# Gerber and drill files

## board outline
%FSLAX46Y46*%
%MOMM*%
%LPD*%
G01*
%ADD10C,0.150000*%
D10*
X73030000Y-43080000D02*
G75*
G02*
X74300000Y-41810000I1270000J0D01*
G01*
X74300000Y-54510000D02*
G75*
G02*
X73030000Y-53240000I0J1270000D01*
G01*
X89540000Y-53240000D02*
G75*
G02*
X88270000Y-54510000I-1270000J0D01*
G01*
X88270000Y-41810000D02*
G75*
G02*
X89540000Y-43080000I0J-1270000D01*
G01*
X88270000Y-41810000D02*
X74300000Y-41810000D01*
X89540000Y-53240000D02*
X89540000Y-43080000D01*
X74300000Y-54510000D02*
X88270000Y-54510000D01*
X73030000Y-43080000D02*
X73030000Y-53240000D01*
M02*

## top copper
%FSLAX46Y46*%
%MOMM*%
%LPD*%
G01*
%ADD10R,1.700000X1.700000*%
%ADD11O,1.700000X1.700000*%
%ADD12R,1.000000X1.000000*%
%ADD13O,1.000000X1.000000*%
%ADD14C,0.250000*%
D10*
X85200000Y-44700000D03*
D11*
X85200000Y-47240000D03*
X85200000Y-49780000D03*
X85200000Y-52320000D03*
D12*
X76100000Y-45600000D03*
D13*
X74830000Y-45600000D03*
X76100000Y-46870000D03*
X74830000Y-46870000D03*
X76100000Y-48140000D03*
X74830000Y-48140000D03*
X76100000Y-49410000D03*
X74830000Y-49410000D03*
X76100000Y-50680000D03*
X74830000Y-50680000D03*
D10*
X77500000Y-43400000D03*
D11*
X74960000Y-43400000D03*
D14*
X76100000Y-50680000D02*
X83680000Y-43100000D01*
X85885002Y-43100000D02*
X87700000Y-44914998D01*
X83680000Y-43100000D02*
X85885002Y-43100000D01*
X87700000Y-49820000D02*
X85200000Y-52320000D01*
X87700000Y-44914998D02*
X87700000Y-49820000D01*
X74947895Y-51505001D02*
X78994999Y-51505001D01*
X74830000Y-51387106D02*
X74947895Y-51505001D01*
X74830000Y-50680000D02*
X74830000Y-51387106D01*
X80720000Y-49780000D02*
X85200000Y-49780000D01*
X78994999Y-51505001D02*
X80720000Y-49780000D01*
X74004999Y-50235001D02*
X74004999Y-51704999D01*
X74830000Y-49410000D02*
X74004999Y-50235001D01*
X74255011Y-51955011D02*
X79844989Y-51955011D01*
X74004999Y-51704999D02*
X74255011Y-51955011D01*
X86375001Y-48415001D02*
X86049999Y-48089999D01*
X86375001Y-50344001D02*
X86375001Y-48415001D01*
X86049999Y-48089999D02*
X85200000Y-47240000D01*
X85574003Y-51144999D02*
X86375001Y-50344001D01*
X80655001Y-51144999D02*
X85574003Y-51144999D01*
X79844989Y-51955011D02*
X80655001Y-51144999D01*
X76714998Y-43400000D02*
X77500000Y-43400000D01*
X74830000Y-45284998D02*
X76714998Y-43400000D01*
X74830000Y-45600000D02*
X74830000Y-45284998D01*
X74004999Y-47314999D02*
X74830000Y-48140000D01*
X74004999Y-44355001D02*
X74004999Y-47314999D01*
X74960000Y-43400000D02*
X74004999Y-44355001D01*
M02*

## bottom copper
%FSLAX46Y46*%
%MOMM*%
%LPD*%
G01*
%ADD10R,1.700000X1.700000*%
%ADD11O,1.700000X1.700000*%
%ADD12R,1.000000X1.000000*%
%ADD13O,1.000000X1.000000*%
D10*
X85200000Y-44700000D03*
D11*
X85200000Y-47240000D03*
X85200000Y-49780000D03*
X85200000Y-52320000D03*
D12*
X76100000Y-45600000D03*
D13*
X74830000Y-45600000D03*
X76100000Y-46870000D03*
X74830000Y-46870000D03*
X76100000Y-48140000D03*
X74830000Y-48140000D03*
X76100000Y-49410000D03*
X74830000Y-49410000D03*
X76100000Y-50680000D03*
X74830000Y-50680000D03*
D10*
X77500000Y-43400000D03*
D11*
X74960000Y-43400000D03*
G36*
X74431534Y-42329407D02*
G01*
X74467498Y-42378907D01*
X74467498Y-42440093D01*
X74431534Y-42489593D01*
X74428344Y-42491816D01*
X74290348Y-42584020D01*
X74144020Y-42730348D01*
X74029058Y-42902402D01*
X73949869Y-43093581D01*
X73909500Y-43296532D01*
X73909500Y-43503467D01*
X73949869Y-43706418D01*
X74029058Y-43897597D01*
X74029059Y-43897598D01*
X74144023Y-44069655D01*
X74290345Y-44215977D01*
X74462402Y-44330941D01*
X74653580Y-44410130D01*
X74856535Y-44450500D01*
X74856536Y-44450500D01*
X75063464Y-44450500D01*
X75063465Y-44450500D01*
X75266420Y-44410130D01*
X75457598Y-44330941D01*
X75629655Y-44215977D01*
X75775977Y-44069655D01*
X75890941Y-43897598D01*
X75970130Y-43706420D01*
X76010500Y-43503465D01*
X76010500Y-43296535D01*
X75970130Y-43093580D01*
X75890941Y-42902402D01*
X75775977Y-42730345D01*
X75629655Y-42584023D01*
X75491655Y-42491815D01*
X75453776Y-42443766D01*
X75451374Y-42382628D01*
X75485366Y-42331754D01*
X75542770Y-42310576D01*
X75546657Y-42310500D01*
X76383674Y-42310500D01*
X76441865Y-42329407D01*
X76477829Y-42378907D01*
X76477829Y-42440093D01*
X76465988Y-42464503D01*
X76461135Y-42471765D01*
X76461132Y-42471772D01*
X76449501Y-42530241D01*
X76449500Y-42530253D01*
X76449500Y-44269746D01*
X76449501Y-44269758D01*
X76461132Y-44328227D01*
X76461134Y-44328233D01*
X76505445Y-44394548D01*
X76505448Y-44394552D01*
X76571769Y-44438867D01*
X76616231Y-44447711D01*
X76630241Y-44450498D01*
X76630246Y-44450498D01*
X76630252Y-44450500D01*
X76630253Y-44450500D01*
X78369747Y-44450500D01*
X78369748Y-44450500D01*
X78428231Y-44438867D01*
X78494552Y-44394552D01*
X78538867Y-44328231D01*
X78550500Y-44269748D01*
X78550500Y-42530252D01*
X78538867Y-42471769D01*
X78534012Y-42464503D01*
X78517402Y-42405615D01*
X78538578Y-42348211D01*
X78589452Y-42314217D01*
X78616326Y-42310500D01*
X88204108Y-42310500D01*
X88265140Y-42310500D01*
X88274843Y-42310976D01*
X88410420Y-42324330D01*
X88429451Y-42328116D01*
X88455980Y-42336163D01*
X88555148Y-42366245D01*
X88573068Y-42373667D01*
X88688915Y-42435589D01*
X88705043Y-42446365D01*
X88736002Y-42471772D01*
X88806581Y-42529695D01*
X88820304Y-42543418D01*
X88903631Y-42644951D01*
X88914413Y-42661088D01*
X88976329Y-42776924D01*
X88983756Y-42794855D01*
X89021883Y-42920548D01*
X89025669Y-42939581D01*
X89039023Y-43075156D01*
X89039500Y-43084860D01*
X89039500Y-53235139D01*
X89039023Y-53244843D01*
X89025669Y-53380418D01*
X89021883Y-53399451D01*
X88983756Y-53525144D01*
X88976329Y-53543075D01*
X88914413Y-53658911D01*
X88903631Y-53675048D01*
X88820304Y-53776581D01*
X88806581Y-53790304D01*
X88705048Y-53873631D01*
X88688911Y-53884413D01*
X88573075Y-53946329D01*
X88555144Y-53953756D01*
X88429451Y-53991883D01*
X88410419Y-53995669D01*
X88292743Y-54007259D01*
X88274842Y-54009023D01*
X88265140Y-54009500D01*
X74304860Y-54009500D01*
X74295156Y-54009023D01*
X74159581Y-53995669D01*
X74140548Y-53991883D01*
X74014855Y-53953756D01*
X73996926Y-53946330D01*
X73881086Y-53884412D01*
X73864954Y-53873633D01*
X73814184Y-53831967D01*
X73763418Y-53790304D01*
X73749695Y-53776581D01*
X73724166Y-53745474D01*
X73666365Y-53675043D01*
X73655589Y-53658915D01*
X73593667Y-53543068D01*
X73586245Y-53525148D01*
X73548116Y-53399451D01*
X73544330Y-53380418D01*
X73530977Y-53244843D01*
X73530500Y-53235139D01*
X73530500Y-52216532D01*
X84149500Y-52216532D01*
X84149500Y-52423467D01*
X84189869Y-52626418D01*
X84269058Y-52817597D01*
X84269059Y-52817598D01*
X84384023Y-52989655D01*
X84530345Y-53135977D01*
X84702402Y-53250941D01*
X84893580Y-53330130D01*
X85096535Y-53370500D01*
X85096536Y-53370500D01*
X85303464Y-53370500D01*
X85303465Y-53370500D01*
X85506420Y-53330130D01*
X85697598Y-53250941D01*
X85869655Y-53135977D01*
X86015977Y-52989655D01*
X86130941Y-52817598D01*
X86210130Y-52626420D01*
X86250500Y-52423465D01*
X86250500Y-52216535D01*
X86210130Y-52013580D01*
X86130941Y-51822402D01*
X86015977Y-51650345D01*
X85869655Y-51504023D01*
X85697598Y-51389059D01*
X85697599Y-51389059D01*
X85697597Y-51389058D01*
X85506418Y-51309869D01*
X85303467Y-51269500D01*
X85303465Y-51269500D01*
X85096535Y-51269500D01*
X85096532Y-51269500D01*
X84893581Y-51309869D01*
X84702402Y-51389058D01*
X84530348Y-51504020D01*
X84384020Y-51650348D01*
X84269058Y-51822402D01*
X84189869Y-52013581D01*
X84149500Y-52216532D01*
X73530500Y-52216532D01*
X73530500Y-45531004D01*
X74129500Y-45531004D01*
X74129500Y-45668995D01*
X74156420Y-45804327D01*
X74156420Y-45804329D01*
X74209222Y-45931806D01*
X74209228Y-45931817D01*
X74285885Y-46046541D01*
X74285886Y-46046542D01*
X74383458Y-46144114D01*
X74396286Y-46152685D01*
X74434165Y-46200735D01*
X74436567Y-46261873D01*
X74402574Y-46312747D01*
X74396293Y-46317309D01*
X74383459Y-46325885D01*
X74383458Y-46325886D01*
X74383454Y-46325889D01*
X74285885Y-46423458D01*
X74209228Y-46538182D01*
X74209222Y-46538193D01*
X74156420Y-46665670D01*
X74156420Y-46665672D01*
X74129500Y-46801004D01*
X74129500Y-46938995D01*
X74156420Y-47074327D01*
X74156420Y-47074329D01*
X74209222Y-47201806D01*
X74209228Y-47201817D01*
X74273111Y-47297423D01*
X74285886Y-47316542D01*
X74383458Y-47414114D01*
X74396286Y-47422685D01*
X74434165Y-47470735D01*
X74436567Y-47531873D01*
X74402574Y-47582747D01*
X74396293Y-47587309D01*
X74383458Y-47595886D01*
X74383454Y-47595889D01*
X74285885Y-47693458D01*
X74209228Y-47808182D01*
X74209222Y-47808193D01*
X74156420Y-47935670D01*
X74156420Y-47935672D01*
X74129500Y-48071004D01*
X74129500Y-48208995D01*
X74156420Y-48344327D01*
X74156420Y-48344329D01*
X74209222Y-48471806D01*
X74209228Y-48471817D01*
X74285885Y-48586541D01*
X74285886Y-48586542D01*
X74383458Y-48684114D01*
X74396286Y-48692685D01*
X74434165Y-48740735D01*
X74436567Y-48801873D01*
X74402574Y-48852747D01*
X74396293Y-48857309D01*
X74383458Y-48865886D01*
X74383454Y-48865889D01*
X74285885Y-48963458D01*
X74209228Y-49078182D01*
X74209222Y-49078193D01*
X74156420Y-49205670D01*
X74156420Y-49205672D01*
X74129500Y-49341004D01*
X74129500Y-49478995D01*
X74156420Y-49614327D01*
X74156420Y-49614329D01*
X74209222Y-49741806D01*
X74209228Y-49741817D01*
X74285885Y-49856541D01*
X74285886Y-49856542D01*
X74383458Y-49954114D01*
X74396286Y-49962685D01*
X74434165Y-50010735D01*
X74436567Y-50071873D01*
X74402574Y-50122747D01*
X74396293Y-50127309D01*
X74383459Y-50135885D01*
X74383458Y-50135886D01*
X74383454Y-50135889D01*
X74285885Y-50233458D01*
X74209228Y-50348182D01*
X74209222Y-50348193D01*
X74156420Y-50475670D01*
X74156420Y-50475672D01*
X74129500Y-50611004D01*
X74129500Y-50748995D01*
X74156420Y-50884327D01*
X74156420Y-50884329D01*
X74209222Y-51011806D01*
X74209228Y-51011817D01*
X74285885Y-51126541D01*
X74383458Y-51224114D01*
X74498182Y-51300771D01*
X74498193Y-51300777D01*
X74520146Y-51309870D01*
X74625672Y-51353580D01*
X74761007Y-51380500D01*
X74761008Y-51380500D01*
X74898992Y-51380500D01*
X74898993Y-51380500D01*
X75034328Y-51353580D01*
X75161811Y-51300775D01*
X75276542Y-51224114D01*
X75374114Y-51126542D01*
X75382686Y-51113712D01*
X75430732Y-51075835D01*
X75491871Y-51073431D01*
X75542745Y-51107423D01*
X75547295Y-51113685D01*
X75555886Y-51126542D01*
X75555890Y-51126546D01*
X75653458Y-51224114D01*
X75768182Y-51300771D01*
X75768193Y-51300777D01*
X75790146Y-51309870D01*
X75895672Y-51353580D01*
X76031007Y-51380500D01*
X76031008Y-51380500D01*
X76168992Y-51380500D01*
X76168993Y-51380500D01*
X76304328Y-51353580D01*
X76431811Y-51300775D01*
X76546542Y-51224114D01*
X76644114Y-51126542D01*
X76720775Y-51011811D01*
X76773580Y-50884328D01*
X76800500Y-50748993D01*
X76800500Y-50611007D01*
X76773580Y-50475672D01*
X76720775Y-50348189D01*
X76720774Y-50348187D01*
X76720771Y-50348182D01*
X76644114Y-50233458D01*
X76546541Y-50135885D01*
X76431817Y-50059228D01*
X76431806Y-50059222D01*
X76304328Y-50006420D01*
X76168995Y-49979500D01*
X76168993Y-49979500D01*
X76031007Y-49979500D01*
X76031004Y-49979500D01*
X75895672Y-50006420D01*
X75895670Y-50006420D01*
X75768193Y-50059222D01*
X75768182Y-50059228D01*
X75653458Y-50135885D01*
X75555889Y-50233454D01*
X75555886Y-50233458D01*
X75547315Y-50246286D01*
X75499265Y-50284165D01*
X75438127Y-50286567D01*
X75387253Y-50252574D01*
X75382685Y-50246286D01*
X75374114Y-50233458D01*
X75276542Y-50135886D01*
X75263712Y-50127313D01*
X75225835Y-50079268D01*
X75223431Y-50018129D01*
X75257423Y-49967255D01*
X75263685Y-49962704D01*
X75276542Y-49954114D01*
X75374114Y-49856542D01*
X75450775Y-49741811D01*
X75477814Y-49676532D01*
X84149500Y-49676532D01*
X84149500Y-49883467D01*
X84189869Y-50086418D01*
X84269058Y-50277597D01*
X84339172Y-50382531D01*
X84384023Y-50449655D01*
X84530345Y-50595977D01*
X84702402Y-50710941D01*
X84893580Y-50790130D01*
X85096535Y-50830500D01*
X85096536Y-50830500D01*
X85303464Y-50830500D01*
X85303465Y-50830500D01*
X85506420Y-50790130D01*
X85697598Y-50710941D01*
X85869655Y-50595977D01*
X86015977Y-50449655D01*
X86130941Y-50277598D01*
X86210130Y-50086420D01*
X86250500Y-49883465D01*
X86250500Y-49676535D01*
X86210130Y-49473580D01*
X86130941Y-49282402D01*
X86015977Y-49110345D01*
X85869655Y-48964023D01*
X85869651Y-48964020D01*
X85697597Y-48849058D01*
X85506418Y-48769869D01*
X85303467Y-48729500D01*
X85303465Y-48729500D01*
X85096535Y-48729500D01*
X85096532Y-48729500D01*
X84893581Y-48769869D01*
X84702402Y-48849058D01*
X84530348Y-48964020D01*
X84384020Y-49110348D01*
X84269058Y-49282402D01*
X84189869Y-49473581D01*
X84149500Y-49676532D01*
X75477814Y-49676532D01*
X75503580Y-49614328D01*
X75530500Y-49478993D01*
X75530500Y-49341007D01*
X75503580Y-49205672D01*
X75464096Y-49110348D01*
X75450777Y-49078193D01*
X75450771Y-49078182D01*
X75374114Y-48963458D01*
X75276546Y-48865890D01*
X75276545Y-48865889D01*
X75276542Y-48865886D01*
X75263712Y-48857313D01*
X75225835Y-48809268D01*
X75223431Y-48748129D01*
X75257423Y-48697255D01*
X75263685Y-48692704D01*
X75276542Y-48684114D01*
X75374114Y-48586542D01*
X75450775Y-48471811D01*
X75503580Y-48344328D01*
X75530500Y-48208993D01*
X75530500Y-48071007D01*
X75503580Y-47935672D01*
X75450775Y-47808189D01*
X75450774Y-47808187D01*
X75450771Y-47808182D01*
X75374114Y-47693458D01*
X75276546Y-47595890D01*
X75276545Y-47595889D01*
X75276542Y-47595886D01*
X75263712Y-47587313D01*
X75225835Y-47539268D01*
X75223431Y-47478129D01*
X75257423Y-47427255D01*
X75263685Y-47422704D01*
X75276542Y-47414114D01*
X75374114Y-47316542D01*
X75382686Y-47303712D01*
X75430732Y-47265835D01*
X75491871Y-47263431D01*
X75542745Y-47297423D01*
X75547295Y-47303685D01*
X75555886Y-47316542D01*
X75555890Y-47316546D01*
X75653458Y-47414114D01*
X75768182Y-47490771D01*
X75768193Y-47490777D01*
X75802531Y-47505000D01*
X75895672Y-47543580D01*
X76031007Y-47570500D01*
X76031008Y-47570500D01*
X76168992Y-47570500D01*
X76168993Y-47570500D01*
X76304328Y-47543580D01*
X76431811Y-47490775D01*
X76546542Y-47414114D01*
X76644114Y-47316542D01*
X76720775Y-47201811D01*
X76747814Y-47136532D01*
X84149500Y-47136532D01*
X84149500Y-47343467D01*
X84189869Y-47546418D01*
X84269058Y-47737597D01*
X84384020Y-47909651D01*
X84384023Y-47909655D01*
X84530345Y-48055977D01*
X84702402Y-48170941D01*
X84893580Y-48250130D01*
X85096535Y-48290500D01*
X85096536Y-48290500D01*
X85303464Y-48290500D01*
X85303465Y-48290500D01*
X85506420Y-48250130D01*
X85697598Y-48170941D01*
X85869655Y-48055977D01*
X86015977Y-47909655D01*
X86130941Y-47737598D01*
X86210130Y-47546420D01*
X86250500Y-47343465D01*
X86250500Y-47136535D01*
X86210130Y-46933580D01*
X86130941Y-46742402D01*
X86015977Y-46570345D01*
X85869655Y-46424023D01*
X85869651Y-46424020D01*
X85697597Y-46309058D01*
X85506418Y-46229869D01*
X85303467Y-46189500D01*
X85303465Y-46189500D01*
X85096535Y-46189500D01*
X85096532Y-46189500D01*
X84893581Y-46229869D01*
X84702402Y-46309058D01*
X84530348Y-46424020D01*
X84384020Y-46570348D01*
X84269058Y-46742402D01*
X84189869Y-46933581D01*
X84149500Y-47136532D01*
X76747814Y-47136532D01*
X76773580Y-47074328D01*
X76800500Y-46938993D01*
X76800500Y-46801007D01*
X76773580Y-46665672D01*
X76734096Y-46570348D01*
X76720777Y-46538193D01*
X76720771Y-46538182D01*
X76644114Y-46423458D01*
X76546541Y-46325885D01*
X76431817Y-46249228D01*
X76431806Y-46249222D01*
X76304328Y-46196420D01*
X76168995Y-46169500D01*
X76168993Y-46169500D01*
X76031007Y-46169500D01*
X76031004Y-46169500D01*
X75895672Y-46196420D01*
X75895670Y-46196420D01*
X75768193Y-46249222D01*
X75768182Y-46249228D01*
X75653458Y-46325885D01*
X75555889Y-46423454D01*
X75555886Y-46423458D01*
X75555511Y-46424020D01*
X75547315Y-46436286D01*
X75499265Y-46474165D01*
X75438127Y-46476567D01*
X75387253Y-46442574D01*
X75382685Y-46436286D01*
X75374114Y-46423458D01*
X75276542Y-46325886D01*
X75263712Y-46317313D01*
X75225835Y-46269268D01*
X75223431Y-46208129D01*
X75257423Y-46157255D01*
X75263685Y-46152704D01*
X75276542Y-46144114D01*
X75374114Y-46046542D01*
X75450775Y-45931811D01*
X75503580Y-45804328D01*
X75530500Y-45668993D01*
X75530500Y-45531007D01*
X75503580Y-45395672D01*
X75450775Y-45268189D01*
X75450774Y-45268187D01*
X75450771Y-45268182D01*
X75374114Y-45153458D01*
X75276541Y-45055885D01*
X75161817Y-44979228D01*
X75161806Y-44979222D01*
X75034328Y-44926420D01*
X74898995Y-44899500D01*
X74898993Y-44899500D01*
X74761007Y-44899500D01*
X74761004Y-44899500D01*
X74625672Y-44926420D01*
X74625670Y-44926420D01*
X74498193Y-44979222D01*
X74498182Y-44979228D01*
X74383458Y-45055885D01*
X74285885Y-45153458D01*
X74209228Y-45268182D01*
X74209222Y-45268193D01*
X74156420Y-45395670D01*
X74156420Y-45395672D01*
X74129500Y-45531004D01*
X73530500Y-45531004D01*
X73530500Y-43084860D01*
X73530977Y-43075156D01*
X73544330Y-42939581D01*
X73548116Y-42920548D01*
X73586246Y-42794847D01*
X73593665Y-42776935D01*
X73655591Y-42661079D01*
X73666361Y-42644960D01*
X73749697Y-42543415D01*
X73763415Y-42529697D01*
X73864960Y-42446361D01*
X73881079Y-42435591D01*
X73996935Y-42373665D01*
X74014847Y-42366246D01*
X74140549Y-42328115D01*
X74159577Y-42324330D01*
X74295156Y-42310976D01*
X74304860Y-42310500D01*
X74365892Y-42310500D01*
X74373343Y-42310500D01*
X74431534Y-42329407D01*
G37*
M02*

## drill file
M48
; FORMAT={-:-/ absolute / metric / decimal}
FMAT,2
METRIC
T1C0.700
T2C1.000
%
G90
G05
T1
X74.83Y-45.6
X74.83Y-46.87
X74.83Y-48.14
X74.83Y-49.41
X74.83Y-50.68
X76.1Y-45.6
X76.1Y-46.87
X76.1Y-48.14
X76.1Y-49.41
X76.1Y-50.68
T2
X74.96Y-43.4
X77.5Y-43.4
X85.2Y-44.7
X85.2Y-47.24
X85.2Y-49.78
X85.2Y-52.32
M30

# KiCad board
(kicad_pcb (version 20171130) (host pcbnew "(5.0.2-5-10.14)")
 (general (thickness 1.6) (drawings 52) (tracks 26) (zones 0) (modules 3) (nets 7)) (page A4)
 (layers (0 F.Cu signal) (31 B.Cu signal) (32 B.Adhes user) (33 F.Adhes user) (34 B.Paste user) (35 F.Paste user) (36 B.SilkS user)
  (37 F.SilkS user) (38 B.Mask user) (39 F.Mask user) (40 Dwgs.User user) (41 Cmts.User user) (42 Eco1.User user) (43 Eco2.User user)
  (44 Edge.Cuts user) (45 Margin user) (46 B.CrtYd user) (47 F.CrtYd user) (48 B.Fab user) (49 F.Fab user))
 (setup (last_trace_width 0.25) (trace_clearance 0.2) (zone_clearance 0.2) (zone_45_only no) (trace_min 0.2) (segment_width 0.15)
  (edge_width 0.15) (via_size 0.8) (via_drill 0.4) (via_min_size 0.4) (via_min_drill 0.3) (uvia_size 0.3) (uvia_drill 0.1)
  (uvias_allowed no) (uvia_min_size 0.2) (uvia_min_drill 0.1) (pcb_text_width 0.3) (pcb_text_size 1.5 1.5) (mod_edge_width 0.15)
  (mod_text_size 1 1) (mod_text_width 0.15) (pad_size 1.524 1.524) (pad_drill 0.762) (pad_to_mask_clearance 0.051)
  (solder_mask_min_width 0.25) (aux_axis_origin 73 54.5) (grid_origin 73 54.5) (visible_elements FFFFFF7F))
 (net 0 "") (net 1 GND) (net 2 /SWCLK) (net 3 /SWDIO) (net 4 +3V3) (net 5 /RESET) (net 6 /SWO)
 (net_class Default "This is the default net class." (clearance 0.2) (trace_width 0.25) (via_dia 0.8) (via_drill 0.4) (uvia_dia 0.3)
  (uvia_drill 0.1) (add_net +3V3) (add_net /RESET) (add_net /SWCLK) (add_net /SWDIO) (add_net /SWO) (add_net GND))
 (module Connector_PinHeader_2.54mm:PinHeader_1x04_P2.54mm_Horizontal (layer F.Cu) (at 85.2 44.7)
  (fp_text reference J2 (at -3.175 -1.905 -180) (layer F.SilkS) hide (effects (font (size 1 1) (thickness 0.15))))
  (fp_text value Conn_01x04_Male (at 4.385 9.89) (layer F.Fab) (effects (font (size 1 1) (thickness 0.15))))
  (pad 1 thru_hole rect (at 0 0) (size 1.7 1.7) (drill 1) (layers *.Cu *.Mask) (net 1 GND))
  (pad 2 thru_hole oval (at 0 2.54) (size 1.7 1.7) (drill 1) (layers *.Cu *.Mask) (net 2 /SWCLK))
  (pad 3 thru_hole oval (at 0 5.08) (size 1.7 1.7) (drill 1) (layers *.Cu *.Mask) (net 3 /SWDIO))
  (pad 4 thru_hole oval (at 0 7.62) (size 1.7 1.7) (drill 1) (layers *.Cu *.Mask) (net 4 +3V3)))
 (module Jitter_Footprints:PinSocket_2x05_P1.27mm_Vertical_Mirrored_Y (layer F.Cu) (at 76.1 45.6)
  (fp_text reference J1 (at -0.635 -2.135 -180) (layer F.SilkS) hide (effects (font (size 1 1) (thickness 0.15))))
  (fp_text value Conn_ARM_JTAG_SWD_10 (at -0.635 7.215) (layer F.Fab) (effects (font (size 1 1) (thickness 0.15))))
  (pad 9 thru_hole rect (at 0 0) (size 1 1) (drill 0.7) (layers *.Cu *.Mask) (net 1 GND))
  (pad 10 thru_hole oval (at -1.27 0) (size 1 1) (drill 0.7) (layers *.Cu *.Mask) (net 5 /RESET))
  (pad 7 thru_hole oval (at 0 1.27) (size 1 1) (drill 0.7) (layers *.Cu *.Mask))
  (pad 8 thru_hole oval (at -1.27 1.27) (size 1 1) (drill 0.7) (layers *.Cu *.Mask))
  (pad 5 thru_hole oval (at 0 2.54) (size 1 1) (drill 0.7) (layers *.Cu *.Mask) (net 1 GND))
  (pad 6 thru_hole oval (at -1.27 2.54) (size 1 1) (drill 0.7) (layers *.Cu *.Mask) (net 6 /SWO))
  (pad 3 thru_hole oval (at 0 3.81) (size 1 1) (drill 0.7) (layers *.Cu *.Mask) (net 1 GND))
  (pad 4 thru_hole oval (at -1.27 3.81) (size 1 1) (drill 0.7) (layers *.Cu *.Mask) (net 2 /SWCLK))
  (pad 1 thru_hole oval (at 0 5.08) (size 1 1) (drill 0.7) (layers *.Cu *.Mask) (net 4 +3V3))
  (pad 2 thru_hole oval (at -1.27 5.08) (size 1 1) (drill 0.7) (layers *.Cu *.Mask) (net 3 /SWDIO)))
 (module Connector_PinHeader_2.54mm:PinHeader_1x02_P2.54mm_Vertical (layer F.Cu) (at 77.5 43.4 270)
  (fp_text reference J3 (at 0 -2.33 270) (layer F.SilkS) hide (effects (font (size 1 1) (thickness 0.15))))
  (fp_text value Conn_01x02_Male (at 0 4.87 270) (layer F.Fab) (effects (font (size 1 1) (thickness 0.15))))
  (pad 1 thru_hole rect (at 0 0 270) (size 1.7 1.7) (drill 1) (layers *.Cu *.Mask) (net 5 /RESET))
  (pad 2 thru_hole oval (at 0 2.54 270) (size 1.7 1.7) (drill 1) (layers *.Cu *.Mask) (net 6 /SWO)))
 (gr_arc (start 74.3 43.08) (end 74.3 41.81) (angle -90) (layer Edge.Cuts) (width 0.15))
 (gr_arc (start 74.3 53.24) (end 73.03 53.24) (angle -90) (layer Edge.Cuts) (width 0.15))
 (gr_arc (start 88.27 53.24) (end 88.27 54.51) (angle -90) (layer Edge.Cuts) (width 0.15))
 (gr_arc (start 88.27 43.08) (end 89.54 43.08) (angle -90) (layer Edge.Cuts) (width 0.15))
 (gr_line (start 88.27 41.81) (end 74.3 41.81) (layer Edge.Cuts) (width 0.15))
 (gr_line (start 89.54 53.24) (end 89.54 43.08) (layer Edge.Cuts) (width 0.15))
 (gr_line (start 74.3 54.51) (end 88.27 54.51) (layer Edge.Cuts) (width 0.15))
 (gr_line (start 73.03 43.08) (end 73.03 53.24) (layer Edge.Cuts) (width 0.15))
 (segment (start 76.1 50.68) (end 83.68 43.1) (width 0.25) (layer F.Cu) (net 4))
 (segment (start 85.885002 43.1) (end 87.7 44.914998) (width 0.25) (layer F.Cu) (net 4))
 (segment (start 83.68 43.1) (end 85.885002 43.1) (width 0.25) (layer F.Cu) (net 4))
 (segment (start 87.7 49.82) (end 85.2 52.32) (width 0.25) (layer F.Cu) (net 4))
 (segment (start 87.7 44.914998) (end 87.7 49.82) (width 0.25) (layer F.Cu) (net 4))
 (segment (start 74.947895 51.505001) (end 78.994999 51.505001) (width 0.25) (layer F.Cu) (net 3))
 (segment (start 74.83 51.387106) (end 74.947895 51.505001) (width 0.25) (layer F.Cu) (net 3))
 (segment (start 74.83 50.68) (end 74.83 51.387106) (width 0.25) (layer F.Cu) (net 3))
 (segment (start 80.72 49.78) (end 85.2 49.78) (width 0.25) (layer F.Cu) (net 3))
 (segment (start 78.994999 51.505001) (end 80.72 49.78) (width 0.25) (layer F.Cu) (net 3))
 (segment (start 74.004999 50.235001) (end 74.004999 51.704999) (width 0.25) (layer F.Cu) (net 2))
 (segment (start 74.83 49.41) (end 74.004999 50.235001) (width 0.25) (layer F.Cu) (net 2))
 (segment (start 74.255011 51.955011) (end 79.844989 51.955011) (width 0.25) (layer F.Cu) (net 2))
 (segment (start 74.004999 51.704999) (end 74.255011 51.955011) (width 0.25) (layer F.Cu) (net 2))
 (segment (start 86.375001 48.415001) (end 86.049999 48.089999) (width 0.25) (layer F.Cu) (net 2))
 (segment (start 86.375001 50.344001) (end 86.375001 48.415001) (width 0.25) (layer F.Cu) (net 2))
 (segment (start 86.049999 48.089999) (end 85.2 47.24) (width 0.25) (layer F.Cu) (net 2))
 (segment (start 85.574003 51.144999) (end 86.375001 50.344001) (width 0.25) (layer F.Cu) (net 2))
 (segment (start 80.655001 51.144999) (end 85.574003 51.144999) (width 0.25) (layer F.Cu) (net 2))
 (segment (start 79.844989 51.955011) (end 80.655001 51.144999) (width 0.25) (layer F.Cu) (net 2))
 (segment (start 76.714998 43.4) (end 77.5 43.4) (width 0.25) (layer F.Cu) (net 5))
 (segment (start 74.83 45.284998) (end 76.714998 43.4) (width 0.25) (layer F.Cu) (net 5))
 (segment (start 74.83 45.6) (end 74.83 45.284998) (width 0.25) (layer F.Cu) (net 5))
 (segment (start 74.004999 47.314999) (end 74.83 48.14) (width 0.25) (layer F.Cu) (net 6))
 (segment (start 74.004999 44.355001) (end 74.004999 47.314999) (width 0.25) (layer F.Cu) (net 6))
 (segment (start 74.96 43.4) (end 74.004999 44.355001) (width 0.25) (layer F.Cu) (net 6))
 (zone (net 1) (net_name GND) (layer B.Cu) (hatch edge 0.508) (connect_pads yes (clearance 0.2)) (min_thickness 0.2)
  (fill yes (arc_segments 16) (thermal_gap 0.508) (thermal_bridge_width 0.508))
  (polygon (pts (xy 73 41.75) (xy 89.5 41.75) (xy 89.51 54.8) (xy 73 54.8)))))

